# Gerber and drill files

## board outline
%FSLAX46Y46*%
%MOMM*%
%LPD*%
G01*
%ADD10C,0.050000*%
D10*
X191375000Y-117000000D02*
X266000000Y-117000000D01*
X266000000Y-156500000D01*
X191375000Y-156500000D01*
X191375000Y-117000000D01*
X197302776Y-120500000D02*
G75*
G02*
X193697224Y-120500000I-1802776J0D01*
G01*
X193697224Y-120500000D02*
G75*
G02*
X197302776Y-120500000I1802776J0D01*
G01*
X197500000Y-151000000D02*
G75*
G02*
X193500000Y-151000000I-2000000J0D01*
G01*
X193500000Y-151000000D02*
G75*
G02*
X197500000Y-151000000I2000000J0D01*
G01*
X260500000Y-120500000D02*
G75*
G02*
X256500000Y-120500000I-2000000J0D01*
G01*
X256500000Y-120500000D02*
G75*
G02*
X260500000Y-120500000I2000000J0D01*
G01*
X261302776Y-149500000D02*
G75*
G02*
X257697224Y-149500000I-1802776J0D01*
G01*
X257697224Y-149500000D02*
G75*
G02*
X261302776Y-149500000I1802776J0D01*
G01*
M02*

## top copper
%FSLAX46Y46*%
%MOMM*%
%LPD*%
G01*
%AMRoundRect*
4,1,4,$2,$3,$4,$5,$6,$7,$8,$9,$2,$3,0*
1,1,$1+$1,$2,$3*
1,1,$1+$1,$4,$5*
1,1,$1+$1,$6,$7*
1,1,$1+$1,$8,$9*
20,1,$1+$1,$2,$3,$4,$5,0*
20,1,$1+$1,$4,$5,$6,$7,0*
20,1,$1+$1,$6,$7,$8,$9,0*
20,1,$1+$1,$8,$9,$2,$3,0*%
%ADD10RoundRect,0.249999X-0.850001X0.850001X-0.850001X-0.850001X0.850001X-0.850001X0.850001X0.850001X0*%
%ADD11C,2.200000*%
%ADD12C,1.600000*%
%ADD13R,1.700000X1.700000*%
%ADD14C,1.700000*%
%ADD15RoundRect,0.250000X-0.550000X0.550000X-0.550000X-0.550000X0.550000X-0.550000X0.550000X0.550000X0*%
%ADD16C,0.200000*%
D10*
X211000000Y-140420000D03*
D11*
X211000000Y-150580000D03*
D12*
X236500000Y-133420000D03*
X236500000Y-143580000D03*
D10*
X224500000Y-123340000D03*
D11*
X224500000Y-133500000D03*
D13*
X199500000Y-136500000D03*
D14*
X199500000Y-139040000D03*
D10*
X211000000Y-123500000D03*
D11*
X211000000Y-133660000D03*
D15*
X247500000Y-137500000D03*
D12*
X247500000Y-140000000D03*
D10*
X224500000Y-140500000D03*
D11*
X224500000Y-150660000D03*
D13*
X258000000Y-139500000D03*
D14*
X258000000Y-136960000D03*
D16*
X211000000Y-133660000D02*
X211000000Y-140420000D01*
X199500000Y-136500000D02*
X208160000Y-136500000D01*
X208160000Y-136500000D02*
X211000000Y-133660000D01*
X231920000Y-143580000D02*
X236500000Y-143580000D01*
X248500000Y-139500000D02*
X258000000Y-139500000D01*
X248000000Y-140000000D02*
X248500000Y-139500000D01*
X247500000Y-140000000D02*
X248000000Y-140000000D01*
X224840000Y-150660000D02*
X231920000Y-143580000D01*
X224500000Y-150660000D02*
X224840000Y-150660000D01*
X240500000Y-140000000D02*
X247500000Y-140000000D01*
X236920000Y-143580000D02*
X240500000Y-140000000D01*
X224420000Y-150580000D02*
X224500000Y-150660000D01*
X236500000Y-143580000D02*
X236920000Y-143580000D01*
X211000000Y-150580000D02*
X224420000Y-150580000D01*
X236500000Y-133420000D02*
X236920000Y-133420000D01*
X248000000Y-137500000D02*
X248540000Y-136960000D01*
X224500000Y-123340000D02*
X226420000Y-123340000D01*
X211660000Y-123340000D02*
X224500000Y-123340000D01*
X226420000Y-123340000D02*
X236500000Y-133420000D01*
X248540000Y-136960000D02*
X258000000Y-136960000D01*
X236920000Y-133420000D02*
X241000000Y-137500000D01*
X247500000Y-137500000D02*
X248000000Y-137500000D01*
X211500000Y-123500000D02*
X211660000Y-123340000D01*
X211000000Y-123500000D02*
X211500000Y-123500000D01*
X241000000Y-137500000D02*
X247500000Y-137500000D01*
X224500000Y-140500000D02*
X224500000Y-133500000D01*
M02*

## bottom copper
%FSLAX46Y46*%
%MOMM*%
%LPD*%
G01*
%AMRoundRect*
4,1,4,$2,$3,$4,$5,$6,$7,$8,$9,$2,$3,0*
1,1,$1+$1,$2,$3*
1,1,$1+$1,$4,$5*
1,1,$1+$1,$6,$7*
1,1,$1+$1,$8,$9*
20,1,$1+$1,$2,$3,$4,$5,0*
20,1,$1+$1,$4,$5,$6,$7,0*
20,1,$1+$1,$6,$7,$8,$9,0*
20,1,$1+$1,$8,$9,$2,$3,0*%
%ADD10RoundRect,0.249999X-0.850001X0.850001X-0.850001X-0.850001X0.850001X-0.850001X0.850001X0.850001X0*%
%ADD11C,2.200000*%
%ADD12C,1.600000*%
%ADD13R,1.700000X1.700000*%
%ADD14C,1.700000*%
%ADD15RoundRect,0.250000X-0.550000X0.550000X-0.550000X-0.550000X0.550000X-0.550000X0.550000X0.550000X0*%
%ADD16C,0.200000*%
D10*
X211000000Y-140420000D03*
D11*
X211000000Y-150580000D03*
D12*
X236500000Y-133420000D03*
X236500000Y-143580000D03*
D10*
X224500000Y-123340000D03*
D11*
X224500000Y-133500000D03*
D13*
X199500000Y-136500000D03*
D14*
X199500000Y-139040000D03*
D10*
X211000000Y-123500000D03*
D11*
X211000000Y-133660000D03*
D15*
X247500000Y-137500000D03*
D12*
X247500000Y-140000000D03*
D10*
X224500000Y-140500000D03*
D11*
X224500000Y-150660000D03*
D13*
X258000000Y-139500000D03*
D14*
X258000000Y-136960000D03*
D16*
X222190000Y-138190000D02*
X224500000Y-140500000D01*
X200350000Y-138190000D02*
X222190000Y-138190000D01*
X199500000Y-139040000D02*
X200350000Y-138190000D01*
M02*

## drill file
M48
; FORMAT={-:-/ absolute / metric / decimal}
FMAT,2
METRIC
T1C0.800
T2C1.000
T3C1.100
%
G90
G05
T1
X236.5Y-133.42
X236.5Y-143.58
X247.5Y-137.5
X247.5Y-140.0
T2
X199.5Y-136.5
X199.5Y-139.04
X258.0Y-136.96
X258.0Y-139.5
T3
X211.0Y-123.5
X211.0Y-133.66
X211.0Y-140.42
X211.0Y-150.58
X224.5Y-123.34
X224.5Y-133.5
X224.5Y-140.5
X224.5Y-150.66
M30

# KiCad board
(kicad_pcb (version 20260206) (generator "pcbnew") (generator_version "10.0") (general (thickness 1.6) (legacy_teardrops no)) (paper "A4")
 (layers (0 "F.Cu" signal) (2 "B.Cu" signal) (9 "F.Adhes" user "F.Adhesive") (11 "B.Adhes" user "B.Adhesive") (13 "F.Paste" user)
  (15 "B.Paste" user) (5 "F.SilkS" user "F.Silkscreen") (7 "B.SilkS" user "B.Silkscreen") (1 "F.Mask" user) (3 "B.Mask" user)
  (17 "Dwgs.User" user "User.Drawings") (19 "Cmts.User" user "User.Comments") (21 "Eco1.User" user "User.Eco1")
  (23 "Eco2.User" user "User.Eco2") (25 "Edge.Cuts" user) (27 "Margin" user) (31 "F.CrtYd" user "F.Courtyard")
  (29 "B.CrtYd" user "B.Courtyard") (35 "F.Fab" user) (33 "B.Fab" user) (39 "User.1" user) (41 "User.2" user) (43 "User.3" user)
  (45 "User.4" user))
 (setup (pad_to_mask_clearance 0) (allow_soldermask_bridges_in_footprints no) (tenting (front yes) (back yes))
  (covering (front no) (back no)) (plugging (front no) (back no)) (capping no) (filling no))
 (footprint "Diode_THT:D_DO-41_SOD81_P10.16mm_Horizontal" (layer "F.Cu") (at 211 140.42 -90)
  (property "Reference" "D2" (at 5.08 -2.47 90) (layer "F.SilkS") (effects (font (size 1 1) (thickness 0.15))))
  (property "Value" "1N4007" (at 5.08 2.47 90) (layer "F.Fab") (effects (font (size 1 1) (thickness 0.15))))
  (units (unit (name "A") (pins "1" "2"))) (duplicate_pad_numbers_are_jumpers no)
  (pad "1" thru_hole roundrect (at 0 0 270) (size 2.2 2.2) (drill 1.1) (layers "*.Cu" "*.Mask") (remove_unused_layers no)
   (roundrect_rratio 0.113636) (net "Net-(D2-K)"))
  (pad "2" thru_hole circle (at 10.16 0 270) (size 2.2 2.2) (drill 1.1) (layers "*.Cu" "*.Mask") (remove_unused_layers no) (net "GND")))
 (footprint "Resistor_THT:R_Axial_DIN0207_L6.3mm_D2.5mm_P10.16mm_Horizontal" (layer "F.Cu") (at 236.5 133.42 -90)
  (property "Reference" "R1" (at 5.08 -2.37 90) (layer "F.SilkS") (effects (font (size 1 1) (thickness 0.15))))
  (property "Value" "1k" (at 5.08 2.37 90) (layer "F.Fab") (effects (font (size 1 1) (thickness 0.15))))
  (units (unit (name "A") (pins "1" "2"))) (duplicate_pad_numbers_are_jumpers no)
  (pad "1" thru_hole circle (at 0 0 270) (size 1.6 1.6) (drill 0.8) (layers "*.Cu" "*.Mask") (remove_unused_layers no) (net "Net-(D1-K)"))
  (pad "2" thru_hole circle (at 10.16 0 270) (size 1.6 1.6) (drill 0.8) (layers "*.Cu" "*.Mask") (remove_unused_layers no) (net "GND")))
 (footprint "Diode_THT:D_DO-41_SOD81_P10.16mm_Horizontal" (layer "F.Cu") (at 224.5 123.34 -90)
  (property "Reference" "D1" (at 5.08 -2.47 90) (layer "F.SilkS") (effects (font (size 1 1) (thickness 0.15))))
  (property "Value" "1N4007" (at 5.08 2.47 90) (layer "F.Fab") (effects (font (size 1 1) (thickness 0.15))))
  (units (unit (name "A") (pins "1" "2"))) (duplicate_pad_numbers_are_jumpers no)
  (pad "1" thru_hole roundrect (at 0 0 270) (size 2.2 2.2) (drill 1.1) (layers "*.Cu" "*.Mask") (remove_unused_layers no)
   (roundrect_rratio 0.113636) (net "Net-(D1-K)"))
  (pad "2" thru_hole circle (at 10.16 0 270) (size 2.2 2.2) (drill 1.1) (layers "*.Cu" "*.Mask") (remove_unused_layers no)
   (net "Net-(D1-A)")))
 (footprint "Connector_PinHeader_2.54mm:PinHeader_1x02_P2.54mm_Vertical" (layer "F.Cu") (at 199.5 136.5)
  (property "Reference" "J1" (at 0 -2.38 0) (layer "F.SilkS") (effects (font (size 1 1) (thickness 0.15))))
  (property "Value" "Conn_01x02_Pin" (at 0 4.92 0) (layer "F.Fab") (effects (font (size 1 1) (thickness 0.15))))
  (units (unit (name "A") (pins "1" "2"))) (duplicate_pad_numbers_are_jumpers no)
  (pad "1" thru_hole rect (at 0 0) (size 1.7 1.7) (drill 1) (layers "*.Cu" "*.Mask") (remove_unused_layers no) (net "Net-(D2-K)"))
  (pad "2" thru_hole circle (at 0 2.54) (size 1.7 1.7) (drill 1) (layers "*.Cu" "*.Mask") (remove_unused_layers no) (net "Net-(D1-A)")))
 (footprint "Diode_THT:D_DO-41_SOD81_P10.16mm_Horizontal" (layer "F.Cu") (at 211 123.5 -90)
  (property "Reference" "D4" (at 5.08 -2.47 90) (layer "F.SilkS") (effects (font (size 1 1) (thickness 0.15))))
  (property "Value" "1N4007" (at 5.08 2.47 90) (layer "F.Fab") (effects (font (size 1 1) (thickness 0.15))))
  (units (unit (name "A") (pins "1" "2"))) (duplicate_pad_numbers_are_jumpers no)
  (pad "1" thru_hole roundrect (at 0 0 270) (size 2.2 2.2) (drill 1.1) (layers "*.Cu" "*.Mask") (remove_unused_layers no)
   (roundrect_rratio 0.113636) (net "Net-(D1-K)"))
  (pad "2" thru_hole circle (at 10.16 0 270) (size 2.2 2.2) (drill 1.1) (layers "*.Cu" "*.Mask") (remove_unused_layers no)
   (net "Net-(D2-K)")))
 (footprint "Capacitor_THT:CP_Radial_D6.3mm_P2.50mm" (layer "F.Cu") (at 247.5 137.5 -90)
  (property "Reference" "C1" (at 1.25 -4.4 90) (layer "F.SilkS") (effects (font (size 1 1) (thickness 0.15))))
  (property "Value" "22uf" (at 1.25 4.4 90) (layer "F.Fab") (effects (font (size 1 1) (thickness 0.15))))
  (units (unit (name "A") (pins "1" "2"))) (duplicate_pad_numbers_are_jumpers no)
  (pad "1" thru_hole roundrect (at 0 0 270) (size 1.6 1.6) (drill 0.8) (layers "*.Cu" "*.Mask") (remove_unused_layers no)
   (roundrect_rratio 0.15625) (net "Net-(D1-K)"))
  (pad "2" thru_hole circle (at 2.5 0 270) (size 1.6 1.6) (drill 0.8) (layers "*.Cu" "*.Mask") (remove_unused_layers no) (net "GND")))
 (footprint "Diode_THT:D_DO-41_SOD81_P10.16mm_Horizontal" (layer "F.Cu") (at 224.5 140.5 -90)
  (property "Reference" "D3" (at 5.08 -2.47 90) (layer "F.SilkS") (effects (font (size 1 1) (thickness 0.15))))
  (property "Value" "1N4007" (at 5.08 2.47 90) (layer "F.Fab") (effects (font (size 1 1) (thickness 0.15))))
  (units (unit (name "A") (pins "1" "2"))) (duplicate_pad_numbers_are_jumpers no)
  (pad "1" thru_hole roundrect (at 0 0 270) (size 2.2 2.2) (drill 1.1) (layers "*.Cu" "*.Mask") (remove_unused_layers no)
   (roundrect_rratio 0.113636) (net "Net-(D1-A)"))
  (pad "2" thru_hole circle (at 10.16 0 270) (size 2.2 2.2) (drill 1.1) (layers "*.Cu" "*.Mask") (remove_unused_layers no) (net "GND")))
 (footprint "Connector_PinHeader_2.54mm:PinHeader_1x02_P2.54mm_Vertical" (layer "F.Cu") (at 258 139.5 180)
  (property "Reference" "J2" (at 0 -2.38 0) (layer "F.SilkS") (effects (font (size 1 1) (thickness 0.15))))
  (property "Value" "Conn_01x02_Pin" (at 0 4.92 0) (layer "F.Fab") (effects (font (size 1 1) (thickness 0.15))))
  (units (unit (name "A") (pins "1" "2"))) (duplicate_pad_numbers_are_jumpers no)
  (pad "1" thru_hole rect (at 0 0 180) (size 1.7 1.7) (drill 1) (layers "*.Cu" "*.Mask") (remove_unused_layers no) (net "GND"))
  (pad "2" thru_hole circle (at 0 2.54 180) (size 1.7 1.7) (drill 1) (layers "*.Cu" "*.Mask") (remove_unused_layers no) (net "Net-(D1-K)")))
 (gr_rect (start 191.375 117) (end 266 156.5) (stroke (width 0.05) (type default)) (fill no) (layer "Edge.Cuts"))
 (gr_circle (center 195.5 120.5) (end 196.5 122) (stroke (width 0.05) (type default)) (fill no) (layer "Edge.Cuts"))
 (gr_circle (center 195.5 151) (end 195.5 153) (stroke (width 0.05) (type default)) (fill no) (layer "Edge.Cuts"))
 (gr_circle (center 258.5 120.5) (end 258.5 122.5) (stroke (width 0.05) (type default)) (fill no) (layer "Edge.Cuts"))
 (gr_circle (center 259.5 149.5) (end 258.5 151) (stroke (width 0.05) (type default)) (fill no) (layer "Edge.Cuts"))
 (segment (start 211 133.66) (end 211 140.42) (width 0.2) (layer "F.Cu") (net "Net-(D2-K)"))
 (segment (start 199.5 136.5) (end 208.16 136.5) (width 0.2) (layer "F.Cu") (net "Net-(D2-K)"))
 (segment (start 208.16 136.5) (end 211 133.66) (width 0.2) (layer "F.Cu") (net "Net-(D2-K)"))
 (segment (start 231.92 143.58) (end 236.5 143.58) (width 0.2) (layer "F.Cu") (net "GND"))
 (segment (start 248.5 139.5) (end 258 139.5) (width 0.2) (layer "F.Cu") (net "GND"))
 (segment (start 248 140) (end 248.5 139.5) (width 0.2) (layer "F.Cu") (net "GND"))
 (segment (start 247.5 140) (end 248 140) (width 0.2) (layer "F.Cu") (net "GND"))
 (segment (start 224.84 150.66) (end 231.92 143.58) (width 0.2) (layer "F.Cu") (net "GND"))
 (segment (start 224.5 150.66) (end 224.84 150.66) (width 0.2) (layer "F.Cu") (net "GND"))
 (segment (start 240.5 140) (end 247.5 140) (width 0.2) (layer "F.Cu") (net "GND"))
 (segment (start 236.92 143.58) (end 240.5 140) (width 0.2) (layer "F.Cu") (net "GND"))
 (segment (start 224.42 150.58) (end 224.5 150.66) (width 0.2) (layer "F.Cu") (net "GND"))
 (segment (start 236.5 143.58) (end 236.92 143.58) (width 0.2) (layer "F.Cu") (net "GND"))
 (segment (start 211 150.58) (end 224.42 150.58) (width 0.2) (layer "F.Cu") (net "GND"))
 (segment (start 236.5 133.42) (end 236.92 133.42) (width 0.2) (layer "F.Cu") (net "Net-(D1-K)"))
 (segment (start 248 137.5) (end 248.54 136.96) (width 0.2) (layer "F.Cu") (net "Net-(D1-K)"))
 (segment (start 224.5 123.34) (end 226.42 123.34) (width 0.2) (layer "F.Cu") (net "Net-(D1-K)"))
 (segment (start 211.66 123.34) (end 224.5 123.34) (width 0.2) (layer "F.Cu") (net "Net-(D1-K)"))
 (segment (start 226.42 123.34) (end 236.5 133.42) (width 0.2) (layer "F.Cu") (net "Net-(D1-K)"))
 (segment (start 248.54 136.96) (end 258 136.96) (width 0.2) (layer "F.Cu") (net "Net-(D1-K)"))
 (segment (start 236.92 133.42) (end 241 137.5) (width 0.2) (layer "F.Cu") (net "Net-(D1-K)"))
 (segment (start 247.5 137.5) (end 248 137.5) (width 0.2) (layer "F.Cu") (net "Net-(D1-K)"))
 (segment (start 211.5 123.5) (end 211.66 123.34) (width 0.2) (layer "F.Cu") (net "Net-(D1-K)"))
 (segment (start 211 123.5) (end 211.5 123.5) (width 0.2) (layer "F.Cu") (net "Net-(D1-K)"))
 (segment (start 241 137.5) (end 247.5 137.5) (width 0.2) (layer "F.Cu") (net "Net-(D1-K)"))
 (segment (start 224.5 140.5) (end 224.5 133.5) (width 0.2) (layer "F.Cu") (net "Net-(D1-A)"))
 (segment (start 222.19 138.19) (end 224.5 140.5) (width 0.2) (layer "B.Cu") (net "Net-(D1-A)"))
 (segment (start 200.35 138.19) (end 222.19 138.19) (width 0.2) (layer "B.Cu") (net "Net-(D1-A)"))
 (segment (start 199.5 139.04) (end 200.35 138.19) (width 0.2) (layer "B.Cu") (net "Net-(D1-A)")))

